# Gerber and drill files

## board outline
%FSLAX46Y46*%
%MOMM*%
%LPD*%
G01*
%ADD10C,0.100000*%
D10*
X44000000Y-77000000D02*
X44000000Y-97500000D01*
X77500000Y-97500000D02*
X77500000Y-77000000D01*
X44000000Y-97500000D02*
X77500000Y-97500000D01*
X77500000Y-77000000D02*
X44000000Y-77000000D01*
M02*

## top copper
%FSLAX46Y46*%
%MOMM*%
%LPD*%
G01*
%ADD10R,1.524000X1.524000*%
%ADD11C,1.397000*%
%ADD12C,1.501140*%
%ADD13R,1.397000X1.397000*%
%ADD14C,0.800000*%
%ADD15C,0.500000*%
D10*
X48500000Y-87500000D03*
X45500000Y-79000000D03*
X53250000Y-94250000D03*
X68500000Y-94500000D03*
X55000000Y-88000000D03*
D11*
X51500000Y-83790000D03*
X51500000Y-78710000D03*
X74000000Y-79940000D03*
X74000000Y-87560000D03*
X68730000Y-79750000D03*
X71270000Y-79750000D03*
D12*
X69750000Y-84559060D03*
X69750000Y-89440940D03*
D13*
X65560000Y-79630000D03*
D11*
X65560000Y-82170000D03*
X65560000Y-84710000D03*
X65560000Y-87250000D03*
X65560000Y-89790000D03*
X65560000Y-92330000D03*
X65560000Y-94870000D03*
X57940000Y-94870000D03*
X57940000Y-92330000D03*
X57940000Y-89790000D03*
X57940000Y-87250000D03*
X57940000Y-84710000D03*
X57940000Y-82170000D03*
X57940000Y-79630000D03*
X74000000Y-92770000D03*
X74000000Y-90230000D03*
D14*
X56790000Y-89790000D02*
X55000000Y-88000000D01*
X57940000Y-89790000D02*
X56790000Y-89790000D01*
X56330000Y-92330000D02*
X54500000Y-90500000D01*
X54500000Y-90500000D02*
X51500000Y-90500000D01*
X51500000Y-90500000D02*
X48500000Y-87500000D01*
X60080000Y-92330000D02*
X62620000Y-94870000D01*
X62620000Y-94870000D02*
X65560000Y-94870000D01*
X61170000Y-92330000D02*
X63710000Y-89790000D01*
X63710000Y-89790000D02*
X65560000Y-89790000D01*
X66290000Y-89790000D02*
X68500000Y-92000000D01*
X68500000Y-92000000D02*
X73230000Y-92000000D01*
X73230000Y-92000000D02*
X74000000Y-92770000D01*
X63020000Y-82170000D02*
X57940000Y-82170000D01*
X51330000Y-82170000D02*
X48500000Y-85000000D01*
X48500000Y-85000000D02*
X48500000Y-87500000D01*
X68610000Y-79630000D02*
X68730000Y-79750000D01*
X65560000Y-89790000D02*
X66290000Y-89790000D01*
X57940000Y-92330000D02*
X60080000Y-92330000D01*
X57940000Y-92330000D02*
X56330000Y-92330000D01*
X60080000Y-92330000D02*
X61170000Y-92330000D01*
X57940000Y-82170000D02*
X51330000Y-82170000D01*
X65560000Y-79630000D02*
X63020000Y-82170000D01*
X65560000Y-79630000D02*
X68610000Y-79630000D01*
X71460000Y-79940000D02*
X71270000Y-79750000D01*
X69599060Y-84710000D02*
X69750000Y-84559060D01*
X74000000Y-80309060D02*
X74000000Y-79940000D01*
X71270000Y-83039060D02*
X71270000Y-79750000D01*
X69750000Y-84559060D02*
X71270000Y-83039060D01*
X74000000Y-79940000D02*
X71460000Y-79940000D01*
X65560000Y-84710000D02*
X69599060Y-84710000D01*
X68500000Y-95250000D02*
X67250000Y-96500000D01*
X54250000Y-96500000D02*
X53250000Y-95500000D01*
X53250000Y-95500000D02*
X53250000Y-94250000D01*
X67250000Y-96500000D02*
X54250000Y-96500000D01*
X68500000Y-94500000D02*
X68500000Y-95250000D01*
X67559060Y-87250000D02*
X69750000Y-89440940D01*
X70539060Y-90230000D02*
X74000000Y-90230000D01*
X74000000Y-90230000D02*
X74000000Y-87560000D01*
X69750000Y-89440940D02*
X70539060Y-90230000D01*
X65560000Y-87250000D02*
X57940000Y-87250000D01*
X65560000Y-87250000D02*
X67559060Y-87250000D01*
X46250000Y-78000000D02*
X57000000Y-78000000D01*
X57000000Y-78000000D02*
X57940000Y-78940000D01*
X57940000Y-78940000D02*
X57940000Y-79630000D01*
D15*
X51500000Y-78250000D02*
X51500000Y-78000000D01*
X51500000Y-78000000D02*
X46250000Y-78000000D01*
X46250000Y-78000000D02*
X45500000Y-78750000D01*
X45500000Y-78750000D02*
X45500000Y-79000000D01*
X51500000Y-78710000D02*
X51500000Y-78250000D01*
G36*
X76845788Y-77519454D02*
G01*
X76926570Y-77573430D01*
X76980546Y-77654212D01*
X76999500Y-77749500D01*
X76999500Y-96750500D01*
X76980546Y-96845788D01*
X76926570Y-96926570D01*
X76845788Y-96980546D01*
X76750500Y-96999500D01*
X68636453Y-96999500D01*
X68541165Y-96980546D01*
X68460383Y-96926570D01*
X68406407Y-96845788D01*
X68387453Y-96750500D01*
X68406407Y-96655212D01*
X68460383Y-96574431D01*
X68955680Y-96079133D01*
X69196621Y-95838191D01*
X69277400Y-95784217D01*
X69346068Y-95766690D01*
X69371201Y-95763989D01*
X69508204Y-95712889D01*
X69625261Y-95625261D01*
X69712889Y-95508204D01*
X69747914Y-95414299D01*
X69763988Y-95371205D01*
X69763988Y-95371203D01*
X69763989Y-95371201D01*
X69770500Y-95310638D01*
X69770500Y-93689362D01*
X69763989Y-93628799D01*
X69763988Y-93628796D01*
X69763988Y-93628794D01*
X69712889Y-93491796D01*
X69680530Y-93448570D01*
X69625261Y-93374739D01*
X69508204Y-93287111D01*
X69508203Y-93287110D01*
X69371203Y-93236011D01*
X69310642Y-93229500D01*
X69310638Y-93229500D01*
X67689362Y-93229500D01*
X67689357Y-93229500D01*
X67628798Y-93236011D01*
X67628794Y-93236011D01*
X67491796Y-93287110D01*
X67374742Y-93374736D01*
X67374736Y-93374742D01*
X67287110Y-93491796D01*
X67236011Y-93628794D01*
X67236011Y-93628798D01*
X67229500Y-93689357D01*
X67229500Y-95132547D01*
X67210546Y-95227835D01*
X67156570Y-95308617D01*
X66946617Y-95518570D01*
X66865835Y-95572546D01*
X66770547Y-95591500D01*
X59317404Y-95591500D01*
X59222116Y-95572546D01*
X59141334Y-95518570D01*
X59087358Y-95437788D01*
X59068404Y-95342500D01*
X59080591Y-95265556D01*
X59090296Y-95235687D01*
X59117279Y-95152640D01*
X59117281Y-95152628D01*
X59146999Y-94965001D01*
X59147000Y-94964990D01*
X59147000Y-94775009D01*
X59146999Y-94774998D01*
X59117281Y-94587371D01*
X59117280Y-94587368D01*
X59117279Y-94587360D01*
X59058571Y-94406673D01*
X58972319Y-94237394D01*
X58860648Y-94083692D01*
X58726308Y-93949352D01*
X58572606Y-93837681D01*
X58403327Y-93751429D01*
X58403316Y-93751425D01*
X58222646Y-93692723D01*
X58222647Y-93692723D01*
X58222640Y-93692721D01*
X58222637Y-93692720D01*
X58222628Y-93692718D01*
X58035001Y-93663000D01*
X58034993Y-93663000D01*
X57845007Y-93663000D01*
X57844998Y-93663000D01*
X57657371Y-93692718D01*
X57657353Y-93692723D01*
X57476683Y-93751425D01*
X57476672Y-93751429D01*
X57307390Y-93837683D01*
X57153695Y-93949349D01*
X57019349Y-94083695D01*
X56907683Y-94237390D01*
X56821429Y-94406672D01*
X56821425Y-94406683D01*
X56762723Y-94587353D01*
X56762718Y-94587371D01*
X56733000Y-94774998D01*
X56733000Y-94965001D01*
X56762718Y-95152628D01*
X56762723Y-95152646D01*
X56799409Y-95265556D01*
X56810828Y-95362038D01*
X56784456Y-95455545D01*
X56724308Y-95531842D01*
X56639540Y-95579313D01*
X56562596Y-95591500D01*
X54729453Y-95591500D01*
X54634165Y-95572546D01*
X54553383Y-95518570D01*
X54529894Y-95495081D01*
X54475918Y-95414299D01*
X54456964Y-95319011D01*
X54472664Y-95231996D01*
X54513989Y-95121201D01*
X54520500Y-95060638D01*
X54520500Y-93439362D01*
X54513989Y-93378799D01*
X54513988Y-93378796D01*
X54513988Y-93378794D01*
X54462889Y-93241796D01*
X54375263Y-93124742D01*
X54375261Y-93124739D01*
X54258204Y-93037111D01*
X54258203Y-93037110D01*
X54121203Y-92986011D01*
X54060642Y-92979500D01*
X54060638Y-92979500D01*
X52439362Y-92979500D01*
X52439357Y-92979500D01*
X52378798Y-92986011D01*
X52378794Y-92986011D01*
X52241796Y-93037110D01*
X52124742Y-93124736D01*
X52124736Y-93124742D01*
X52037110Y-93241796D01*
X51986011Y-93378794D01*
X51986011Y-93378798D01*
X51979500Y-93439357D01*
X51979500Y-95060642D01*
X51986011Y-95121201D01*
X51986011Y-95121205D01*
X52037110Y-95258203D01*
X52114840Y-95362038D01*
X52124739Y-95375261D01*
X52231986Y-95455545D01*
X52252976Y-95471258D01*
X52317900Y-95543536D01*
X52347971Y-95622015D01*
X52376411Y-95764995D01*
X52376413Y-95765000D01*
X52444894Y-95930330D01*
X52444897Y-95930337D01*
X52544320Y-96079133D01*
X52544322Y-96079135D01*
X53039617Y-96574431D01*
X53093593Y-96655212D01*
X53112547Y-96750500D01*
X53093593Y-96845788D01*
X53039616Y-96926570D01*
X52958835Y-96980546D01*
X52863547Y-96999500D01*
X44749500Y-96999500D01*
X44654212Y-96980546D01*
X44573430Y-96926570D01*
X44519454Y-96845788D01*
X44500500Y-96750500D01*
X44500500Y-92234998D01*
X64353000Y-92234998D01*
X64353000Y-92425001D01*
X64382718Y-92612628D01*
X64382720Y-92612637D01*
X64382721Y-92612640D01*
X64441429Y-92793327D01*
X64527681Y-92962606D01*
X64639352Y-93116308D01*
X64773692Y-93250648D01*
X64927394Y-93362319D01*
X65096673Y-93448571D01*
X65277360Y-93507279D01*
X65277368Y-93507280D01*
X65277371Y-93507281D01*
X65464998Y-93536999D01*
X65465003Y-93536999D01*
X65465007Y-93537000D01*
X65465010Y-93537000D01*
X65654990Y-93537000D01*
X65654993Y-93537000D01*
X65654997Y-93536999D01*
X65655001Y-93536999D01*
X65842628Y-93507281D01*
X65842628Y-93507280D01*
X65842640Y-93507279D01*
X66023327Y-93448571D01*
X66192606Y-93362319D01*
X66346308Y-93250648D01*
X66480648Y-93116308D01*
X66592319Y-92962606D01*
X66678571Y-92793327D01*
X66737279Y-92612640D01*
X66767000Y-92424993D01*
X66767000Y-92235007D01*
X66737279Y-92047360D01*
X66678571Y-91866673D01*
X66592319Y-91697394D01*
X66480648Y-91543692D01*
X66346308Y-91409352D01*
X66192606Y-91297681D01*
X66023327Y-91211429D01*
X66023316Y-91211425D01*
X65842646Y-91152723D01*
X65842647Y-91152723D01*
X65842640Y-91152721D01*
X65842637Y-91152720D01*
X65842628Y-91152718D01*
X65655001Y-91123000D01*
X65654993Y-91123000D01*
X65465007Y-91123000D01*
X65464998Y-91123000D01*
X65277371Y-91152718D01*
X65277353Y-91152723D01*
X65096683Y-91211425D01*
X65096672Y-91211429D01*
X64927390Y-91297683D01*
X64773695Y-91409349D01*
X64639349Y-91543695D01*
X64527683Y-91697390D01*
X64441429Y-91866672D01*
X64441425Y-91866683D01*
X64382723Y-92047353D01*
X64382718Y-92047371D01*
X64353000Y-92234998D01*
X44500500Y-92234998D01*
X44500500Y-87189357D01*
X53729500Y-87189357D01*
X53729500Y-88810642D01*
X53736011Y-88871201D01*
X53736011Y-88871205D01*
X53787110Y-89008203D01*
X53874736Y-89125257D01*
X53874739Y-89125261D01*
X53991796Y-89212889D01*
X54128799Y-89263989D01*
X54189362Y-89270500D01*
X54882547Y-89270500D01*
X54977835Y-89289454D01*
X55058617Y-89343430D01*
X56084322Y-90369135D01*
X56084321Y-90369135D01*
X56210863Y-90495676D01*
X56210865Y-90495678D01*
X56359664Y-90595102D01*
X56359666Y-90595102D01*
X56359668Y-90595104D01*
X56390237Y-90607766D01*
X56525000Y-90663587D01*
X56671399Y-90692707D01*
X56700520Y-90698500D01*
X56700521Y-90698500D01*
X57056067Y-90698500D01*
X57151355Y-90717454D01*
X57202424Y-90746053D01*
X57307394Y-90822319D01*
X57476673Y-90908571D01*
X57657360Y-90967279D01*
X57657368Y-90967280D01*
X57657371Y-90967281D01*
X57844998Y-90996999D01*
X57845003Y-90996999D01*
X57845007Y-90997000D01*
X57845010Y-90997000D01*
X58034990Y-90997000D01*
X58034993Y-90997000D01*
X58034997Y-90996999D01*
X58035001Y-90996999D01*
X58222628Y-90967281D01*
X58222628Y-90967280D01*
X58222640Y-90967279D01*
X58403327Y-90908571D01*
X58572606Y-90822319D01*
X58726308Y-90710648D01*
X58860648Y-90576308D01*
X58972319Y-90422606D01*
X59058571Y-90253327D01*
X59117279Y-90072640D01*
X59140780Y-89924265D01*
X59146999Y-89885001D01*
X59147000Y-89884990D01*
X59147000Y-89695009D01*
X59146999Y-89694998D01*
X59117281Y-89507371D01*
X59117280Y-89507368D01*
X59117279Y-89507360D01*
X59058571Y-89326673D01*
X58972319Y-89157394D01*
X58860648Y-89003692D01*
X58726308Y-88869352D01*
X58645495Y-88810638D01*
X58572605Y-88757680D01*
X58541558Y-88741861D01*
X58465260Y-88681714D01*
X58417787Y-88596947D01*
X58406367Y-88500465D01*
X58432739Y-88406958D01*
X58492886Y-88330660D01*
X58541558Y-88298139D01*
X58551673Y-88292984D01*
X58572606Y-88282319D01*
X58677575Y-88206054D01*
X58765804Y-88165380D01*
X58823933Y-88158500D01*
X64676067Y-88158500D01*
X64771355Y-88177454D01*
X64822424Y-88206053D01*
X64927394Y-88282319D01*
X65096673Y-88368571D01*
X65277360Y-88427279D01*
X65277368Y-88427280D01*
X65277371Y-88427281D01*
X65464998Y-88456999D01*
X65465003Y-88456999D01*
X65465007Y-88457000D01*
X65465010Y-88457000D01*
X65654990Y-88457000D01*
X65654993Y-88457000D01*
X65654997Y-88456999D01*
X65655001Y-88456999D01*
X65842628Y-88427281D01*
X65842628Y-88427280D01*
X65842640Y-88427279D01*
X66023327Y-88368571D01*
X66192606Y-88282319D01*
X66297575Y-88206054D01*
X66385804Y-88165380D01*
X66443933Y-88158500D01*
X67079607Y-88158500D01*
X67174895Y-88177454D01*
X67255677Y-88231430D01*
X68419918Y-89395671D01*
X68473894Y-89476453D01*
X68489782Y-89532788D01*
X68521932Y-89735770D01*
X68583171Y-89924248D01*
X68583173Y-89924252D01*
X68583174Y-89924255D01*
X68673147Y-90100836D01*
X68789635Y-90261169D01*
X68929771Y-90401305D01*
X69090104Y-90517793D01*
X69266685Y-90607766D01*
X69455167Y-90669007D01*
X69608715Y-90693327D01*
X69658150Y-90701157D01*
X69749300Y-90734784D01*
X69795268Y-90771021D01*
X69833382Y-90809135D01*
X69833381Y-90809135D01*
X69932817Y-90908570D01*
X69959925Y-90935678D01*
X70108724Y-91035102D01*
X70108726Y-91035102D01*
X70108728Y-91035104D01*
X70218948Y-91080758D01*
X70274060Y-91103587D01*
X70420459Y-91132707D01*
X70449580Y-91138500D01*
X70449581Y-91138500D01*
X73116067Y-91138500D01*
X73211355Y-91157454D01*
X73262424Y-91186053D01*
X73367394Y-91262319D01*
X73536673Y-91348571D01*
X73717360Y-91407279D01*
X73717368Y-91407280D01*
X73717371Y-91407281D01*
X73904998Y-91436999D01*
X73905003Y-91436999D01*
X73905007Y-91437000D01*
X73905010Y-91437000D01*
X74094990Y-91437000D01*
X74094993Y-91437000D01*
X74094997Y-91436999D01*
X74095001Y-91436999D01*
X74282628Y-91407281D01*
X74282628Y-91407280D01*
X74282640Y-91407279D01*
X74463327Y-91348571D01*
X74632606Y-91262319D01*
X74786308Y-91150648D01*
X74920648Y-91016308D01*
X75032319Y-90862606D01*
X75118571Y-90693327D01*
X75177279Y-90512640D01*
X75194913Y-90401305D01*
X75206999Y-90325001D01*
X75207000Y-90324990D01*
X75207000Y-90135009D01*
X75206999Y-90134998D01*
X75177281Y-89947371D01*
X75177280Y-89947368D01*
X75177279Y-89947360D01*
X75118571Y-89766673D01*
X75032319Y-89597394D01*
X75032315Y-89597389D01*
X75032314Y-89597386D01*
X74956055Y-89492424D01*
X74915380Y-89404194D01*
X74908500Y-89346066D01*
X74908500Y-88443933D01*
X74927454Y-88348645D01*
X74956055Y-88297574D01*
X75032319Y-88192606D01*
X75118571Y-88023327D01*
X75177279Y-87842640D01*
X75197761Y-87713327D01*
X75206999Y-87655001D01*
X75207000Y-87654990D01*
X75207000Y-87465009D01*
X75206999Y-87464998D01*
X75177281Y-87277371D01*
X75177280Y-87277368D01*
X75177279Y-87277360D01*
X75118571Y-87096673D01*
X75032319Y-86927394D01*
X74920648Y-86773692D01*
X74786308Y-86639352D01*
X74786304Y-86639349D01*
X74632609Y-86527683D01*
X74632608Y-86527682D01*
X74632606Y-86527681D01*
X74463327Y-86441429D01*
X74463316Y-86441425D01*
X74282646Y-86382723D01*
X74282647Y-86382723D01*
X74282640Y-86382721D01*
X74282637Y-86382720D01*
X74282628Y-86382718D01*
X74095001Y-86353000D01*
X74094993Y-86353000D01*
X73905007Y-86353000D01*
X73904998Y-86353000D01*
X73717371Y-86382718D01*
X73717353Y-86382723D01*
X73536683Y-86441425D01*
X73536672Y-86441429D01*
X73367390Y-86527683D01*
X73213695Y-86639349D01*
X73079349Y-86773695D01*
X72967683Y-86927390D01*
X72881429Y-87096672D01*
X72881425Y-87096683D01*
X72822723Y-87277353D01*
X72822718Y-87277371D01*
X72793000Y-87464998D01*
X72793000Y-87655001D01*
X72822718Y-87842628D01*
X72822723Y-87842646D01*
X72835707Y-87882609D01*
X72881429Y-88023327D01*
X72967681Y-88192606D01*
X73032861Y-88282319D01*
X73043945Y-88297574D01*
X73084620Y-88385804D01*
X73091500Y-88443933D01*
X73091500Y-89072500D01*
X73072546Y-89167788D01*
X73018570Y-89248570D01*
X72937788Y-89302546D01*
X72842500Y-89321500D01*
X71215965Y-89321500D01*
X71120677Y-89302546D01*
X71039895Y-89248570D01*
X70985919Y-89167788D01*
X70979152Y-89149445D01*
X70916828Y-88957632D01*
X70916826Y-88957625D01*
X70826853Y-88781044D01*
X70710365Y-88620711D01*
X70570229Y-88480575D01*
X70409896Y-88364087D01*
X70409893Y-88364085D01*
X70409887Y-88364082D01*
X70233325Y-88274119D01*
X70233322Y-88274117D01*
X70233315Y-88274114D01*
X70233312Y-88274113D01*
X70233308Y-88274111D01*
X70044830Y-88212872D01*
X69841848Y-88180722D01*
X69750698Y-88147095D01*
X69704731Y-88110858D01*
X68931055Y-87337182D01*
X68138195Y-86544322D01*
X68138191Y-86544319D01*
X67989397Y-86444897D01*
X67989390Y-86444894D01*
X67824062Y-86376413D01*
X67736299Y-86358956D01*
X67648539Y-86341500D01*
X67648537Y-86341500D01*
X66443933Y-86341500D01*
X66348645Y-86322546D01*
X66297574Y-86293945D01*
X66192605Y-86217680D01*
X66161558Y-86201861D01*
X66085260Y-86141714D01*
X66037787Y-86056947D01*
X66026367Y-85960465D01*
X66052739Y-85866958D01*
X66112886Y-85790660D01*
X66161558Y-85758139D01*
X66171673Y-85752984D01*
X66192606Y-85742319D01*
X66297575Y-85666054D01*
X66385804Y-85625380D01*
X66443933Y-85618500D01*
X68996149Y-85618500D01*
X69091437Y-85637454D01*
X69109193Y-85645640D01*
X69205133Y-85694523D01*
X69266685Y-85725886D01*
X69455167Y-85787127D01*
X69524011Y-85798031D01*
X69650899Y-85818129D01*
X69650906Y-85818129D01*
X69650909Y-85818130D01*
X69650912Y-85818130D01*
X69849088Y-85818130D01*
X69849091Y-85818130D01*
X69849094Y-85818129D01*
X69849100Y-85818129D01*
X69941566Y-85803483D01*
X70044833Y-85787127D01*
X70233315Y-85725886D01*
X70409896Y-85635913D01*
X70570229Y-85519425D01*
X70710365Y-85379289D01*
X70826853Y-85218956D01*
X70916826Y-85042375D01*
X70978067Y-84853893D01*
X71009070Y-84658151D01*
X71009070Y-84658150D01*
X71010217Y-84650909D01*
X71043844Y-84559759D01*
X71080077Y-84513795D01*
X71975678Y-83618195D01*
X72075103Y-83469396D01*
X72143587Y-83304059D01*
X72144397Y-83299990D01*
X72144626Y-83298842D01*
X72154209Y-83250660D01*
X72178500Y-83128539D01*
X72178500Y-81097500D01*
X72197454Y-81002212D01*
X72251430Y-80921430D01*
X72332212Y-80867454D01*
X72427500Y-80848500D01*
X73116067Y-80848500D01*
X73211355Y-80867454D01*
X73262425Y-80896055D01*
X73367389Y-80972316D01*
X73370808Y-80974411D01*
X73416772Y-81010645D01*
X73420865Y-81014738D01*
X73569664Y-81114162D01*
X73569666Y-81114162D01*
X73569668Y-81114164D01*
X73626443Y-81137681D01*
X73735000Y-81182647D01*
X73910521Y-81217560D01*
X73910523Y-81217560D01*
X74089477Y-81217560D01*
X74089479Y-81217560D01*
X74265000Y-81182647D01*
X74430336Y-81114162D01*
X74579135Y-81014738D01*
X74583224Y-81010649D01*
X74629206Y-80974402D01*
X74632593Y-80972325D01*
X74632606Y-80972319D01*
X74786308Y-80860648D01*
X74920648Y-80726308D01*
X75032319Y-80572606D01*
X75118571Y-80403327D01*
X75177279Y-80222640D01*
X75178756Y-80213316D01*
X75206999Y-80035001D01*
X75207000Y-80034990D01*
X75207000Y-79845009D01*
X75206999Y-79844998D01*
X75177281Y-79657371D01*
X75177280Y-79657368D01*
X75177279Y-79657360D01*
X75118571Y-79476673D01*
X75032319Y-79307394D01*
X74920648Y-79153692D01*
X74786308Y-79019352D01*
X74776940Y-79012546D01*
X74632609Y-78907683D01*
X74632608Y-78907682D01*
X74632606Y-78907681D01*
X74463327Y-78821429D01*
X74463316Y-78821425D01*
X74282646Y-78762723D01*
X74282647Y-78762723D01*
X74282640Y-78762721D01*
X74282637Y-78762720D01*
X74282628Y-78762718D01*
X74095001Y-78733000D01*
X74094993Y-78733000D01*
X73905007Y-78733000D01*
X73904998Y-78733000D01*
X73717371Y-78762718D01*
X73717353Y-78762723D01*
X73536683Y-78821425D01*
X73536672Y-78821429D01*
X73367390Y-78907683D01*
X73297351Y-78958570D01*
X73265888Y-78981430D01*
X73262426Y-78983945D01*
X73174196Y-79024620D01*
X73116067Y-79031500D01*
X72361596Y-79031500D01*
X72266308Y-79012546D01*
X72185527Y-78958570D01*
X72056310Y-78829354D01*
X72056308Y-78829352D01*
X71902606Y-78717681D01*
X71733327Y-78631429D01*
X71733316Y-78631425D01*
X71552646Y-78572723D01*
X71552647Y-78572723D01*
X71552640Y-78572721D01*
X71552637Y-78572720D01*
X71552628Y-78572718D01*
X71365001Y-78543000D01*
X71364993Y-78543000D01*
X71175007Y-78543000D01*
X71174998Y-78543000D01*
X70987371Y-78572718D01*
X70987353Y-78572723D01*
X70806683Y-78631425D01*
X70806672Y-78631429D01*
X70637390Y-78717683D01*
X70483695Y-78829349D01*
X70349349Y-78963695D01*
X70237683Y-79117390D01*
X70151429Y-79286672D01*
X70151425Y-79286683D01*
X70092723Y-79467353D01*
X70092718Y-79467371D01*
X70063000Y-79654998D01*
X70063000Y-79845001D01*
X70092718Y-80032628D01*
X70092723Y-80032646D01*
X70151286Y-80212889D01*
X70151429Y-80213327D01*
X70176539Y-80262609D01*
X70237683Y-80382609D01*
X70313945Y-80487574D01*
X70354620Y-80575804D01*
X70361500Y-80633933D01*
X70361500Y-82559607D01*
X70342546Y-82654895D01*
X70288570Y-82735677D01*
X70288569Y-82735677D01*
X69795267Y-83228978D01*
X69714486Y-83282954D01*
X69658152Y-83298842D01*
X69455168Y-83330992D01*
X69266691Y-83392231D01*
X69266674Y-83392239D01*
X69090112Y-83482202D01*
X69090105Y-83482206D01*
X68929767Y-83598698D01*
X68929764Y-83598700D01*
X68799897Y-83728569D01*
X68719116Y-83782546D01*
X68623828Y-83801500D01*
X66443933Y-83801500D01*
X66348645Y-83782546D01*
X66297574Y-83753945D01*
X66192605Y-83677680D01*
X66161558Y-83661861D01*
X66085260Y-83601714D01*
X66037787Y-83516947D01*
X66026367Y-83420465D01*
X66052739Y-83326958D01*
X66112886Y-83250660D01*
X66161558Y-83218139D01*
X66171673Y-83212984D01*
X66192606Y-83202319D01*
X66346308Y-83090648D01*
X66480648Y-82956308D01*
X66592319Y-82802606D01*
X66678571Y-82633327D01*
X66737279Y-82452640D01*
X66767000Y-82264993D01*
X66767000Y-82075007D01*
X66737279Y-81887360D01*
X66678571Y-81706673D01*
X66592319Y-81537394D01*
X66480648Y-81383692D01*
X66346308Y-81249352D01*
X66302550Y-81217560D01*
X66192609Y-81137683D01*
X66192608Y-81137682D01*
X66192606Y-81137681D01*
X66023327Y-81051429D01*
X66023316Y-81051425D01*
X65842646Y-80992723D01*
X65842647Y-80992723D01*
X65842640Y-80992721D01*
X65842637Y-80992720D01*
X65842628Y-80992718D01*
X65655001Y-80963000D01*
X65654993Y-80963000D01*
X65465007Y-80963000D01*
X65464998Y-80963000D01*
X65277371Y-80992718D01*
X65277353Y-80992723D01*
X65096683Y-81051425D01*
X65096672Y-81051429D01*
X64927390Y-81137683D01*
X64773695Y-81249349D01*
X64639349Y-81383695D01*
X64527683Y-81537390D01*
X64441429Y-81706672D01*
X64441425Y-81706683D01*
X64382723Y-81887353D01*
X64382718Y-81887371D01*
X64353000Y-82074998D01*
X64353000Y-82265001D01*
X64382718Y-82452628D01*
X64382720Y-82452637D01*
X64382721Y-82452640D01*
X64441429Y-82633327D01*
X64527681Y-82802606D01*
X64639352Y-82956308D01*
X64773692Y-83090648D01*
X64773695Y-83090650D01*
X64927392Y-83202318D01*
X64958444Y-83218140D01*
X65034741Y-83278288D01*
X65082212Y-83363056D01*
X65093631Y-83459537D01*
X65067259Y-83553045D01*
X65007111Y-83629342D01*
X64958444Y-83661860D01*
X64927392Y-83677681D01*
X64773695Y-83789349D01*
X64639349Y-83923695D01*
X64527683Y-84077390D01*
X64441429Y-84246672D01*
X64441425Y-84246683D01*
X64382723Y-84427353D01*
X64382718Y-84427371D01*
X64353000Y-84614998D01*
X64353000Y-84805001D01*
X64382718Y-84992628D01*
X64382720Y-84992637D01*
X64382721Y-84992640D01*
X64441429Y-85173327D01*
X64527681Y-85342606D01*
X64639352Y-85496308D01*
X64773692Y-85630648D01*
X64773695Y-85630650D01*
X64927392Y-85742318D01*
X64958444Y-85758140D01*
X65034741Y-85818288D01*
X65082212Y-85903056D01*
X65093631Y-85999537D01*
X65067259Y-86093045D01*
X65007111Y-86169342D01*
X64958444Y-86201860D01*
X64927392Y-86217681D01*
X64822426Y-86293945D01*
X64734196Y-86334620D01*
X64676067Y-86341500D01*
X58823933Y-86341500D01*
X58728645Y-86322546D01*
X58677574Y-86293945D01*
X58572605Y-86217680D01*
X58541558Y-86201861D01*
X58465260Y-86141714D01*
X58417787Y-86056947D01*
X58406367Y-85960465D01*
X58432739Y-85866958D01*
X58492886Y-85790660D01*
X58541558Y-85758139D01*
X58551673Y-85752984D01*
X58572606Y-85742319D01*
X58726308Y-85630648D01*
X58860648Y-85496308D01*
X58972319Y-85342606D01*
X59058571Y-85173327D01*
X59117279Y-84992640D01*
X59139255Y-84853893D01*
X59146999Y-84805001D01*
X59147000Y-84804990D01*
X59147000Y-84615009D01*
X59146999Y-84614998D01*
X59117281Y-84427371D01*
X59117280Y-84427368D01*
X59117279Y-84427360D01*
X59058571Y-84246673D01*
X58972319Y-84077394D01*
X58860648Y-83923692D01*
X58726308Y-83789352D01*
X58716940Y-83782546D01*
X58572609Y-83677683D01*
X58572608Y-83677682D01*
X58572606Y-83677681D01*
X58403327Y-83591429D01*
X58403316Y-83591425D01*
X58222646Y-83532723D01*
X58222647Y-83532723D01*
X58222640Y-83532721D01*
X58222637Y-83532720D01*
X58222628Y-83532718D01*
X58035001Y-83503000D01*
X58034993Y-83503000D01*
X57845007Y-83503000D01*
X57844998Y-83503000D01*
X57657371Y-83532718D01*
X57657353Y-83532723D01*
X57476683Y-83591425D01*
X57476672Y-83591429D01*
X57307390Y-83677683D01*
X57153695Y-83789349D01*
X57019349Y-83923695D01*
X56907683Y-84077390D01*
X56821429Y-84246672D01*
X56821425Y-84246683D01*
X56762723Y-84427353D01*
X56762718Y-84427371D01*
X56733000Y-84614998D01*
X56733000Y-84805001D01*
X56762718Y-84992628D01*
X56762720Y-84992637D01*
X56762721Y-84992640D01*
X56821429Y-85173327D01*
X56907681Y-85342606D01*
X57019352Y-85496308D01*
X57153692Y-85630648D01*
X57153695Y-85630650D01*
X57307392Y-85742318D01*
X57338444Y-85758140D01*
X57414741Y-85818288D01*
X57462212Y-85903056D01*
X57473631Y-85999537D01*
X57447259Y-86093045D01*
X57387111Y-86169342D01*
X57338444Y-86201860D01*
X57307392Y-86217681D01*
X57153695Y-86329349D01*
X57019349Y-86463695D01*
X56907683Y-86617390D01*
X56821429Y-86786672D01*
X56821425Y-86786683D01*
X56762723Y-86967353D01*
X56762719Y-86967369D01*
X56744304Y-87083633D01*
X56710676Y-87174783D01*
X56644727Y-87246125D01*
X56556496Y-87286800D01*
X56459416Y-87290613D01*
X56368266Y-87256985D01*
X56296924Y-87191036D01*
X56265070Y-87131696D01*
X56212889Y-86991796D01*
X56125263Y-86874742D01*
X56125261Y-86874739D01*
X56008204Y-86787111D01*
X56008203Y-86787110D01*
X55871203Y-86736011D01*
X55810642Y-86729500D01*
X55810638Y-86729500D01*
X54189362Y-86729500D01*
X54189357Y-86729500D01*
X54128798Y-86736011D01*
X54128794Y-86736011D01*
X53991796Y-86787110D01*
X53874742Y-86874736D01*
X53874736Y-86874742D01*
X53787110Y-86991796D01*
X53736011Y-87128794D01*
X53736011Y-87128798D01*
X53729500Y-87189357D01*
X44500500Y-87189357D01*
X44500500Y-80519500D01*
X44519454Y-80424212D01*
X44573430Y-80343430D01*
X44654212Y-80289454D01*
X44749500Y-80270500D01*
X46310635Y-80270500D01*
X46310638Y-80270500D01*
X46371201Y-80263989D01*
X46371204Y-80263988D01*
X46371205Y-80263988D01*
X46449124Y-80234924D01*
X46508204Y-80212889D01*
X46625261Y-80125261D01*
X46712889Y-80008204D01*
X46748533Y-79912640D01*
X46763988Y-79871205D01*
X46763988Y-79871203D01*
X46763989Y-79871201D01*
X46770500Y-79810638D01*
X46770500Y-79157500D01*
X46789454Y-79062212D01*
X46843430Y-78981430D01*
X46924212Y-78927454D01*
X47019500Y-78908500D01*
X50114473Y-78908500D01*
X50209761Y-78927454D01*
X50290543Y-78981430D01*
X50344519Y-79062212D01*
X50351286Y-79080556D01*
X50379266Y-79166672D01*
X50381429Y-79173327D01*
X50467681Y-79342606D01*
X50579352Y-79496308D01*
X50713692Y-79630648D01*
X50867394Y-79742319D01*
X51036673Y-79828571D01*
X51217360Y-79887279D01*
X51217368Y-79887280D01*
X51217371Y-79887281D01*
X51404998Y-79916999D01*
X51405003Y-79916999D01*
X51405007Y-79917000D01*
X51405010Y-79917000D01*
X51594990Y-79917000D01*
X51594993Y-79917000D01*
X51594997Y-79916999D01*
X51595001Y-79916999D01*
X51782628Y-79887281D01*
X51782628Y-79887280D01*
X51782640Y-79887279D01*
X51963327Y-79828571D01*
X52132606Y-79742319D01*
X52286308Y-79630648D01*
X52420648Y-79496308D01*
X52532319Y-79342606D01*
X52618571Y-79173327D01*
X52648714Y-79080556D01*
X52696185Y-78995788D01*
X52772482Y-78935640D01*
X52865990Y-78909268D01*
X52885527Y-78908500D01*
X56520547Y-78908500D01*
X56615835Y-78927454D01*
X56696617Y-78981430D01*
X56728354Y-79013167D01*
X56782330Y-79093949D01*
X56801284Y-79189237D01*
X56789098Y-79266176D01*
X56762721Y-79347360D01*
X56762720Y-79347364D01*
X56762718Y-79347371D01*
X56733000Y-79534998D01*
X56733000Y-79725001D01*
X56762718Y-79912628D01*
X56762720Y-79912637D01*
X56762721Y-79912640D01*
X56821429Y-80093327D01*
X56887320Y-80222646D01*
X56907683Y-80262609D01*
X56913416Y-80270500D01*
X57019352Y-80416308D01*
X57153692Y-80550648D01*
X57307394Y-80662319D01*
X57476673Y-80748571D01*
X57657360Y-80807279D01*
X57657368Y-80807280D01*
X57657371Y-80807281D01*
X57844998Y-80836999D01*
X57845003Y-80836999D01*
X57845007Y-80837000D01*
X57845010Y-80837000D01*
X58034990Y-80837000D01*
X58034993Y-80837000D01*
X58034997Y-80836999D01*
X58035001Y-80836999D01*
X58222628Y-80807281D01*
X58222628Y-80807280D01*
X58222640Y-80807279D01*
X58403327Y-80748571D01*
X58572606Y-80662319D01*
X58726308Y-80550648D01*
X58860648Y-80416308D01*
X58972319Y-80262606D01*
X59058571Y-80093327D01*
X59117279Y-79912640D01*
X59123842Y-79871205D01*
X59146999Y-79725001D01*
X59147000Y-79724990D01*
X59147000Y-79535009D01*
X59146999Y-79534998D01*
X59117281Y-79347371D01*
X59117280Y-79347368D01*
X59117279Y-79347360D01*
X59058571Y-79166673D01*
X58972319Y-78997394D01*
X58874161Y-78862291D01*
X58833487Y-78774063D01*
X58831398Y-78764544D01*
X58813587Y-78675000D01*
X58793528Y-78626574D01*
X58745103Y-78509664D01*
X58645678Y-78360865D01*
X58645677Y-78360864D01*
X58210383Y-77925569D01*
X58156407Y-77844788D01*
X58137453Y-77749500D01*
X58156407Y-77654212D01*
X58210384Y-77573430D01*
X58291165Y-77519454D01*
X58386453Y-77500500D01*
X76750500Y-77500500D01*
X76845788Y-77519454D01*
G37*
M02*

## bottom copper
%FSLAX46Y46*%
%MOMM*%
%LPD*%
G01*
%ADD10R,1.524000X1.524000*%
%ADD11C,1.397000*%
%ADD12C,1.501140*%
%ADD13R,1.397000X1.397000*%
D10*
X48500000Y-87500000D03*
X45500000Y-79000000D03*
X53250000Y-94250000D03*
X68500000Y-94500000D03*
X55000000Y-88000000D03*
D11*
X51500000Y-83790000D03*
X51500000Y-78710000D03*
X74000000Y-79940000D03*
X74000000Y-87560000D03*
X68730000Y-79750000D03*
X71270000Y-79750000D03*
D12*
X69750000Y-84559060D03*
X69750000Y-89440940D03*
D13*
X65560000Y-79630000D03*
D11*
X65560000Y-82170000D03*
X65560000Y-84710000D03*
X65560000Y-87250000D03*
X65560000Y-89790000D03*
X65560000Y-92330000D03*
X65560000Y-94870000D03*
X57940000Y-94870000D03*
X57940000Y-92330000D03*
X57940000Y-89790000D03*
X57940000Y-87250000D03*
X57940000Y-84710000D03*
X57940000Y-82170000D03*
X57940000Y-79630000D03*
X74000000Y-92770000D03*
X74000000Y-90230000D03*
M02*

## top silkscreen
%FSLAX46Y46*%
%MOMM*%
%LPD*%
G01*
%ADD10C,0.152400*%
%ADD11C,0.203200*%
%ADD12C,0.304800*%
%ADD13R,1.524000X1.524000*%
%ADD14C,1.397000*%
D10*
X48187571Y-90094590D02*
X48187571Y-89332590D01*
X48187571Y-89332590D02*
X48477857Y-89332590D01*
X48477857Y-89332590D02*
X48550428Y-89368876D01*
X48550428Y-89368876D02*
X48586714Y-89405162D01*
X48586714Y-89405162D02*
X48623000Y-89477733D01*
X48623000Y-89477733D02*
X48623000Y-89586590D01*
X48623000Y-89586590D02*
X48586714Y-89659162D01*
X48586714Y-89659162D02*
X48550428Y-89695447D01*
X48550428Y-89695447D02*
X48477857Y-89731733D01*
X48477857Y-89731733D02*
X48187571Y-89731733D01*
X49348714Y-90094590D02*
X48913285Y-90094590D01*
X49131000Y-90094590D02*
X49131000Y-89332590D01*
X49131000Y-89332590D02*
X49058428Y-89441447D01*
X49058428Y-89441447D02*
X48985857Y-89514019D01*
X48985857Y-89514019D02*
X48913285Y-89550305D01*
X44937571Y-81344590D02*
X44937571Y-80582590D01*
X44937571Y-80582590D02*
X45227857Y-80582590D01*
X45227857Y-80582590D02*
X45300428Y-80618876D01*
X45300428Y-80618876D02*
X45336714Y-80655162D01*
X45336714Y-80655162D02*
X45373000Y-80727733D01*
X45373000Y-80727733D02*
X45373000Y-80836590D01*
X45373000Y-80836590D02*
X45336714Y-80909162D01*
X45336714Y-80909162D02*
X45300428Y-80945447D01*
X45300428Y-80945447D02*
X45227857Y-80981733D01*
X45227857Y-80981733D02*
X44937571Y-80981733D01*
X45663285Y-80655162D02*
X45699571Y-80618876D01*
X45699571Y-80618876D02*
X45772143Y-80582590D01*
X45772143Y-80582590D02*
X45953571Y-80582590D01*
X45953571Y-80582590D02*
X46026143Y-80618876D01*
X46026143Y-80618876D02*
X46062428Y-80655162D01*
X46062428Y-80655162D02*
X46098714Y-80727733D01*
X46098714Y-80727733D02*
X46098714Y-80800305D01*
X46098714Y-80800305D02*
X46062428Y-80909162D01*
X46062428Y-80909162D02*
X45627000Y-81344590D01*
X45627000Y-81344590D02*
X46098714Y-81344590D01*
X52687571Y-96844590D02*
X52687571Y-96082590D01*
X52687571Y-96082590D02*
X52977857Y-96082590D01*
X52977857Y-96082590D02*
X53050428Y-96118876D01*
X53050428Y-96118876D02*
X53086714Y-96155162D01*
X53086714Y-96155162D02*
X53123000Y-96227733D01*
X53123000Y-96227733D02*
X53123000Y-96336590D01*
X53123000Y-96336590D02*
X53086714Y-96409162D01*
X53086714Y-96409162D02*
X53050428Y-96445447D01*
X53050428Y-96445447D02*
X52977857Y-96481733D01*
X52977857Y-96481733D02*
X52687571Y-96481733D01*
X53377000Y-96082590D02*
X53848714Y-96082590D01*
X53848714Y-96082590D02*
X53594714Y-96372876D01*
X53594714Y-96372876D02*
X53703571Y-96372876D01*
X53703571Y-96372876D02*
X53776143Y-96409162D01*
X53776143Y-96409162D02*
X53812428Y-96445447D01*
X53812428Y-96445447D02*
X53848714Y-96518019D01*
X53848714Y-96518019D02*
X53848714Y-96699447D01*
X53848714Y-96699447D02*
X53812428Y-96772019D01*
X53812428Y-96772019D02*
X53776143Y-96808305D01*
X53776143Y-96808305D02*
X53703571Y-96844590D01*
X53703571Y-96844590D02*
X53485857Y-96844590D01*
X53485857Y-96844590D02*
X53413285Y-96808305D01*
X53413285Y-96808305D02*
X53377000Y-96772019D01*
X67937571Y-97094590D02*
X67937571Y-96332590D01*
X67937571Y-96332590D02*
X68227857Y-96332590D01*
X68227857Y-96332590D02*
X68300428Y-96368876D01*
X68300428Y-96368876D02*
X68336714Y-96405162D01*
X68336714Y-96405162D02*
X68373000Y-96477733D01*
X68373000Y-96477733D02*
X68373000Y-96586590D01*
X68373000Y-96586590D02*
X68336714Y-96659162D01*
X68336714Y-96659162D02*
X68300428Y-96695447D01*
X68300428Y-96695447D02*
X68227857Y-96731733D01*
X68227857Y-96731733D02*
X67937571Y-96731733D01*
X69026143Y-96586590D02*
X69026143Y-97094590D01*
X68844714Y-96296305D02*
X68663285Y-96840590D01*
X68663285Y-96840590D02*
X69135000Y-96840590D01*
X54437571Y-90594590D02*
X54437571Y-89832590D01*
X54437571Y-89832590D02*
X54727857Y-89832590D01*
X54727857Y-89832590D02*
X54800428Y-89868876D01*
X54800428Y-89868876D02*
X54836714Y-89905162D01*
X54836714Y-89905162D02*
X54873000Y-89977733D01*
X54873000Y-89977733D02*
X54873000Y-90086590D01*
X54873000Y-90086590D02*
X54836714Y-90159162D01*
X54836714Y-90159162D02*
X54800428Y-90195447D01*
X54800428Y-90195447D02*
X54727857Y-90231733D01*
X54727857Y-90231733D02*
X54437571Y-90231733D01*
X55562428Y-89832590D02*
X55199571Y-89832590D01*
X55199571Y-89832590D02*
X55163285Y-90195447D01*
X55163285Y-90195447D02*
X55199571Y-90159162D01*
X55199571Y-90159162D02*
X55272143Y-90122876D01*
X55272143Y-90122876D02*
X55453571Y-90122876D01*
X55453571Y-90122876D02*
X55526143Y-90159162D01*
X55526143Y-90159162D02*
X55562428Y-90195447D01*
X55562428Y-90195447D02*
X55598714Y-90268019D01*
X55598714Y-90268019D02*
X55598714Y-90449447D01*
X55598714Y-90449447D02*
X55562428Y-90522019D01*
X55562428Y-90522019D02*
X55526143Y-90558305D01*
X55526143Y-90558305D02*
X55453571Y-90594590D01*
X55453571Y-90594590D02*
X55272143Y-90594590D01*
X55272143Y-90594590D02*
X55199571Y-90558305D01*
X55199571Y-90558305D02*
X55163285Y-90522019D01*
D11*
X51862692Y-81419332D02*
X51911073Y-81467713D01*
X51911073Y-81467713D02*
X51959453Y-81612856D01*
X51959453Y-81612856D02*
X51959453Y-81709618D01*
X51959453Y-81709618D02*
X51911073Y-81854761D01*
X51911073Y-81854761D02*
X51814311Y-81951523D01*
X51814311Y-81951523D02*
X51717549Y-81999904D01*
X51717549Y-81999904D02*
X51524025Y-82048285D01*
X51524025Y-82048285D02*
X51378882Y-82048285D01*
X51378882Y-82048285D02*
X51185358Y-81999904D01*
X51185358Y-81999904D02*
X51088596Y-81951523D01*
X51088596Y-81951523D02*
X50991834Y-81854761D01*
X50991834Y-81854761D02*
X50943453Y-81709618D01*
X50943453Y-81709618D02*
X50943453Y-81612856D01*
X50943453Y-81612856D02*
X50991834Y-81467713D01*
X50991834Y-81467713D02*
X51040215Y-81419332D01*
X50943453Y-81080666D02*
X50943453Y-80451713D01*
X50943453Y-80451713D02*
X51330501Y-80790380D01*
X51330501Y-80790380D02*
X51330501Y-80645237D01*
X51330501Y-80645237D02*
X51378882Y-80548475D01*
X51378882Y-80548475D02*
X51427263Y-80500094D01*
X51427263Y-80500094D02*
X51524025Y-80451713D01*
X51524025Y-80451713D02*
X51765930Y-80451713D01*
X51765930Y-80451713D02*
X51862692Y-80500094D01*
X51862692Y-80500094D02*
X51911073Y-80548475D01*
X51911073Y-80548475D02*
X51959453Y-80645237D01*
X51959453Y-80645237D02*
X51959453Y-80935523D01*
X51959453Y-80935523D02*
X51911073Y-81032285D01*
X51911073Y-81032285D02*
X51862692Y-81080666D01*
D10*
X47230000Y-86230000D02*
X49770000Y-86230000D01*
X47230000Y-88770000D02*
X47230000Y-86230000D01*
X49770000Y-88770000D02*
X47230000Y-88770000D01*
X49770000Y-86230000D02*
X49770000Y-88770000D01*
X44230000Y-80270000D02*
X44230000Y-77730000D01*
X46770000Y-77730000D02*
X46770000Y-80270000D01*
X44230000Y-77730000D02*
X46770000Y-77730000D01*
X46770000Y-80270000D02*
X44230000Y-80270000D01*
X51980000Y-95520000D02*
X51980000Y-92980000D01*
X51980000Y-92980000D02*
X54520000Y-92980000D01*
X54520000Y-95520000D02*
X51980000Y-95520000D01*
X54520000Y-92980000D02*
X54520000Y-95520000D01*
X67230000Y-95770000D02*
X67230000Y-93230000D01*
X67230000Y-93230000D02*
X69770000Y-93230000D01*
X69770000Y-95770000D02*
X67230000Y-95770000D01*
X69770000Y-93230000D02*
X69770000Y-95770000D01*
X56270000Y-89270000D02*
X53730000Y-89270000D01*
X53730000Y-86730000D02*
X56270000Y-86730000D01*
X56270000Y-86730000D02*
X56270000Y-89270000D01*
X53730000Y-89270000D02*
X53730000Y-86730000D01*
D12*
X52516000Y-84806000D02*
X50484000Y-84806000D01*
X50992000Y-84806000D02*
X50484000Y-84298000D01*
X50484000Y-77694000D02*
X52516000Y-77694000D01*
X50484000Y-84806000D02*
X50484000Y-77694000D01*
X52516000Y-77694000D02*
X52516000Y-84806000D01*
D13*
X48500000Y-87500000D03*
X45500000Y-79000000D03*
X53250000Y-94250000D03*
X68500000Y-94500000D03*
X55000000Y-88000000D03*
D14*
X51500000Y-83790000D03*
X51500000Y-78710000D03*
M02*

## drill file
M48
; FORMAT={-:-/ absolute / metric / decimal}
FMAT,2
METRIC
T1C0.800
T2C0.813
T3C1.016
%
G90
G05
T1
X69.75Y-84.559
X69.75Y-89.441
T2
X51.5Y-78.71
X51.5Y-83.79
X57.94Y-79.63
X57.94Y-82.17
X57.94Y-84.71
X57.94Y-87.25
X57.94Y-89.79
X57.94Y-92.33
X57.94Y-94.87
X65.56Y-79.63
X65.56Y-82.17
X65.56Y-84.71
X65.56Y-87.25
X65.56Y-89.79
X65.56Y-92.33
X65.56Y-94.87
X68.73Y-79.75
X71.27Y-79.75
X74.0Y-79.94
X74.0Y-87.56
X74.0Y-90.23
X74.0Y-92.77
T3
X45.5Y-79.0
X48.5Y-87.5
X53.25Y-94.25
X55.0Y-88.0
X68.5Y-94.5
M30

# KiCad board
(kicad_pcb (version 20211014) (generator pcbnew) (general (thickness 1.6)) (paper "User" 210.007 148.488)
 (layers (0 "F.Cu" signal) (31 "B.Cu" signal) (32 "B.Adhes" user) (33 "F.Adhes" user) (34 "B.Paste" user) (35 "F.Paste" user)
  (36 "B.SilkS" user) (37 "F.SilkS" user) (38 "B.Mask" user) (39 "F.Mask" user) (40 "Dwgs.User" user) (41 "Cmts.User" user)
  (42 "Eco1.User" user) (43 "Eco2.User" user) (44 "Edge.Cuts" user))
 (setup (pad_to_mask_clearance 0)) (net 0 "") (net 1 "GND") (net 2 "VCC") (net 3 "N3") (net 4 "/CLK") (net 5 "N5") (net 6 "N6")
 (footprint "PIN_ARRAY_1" (layer "F.Cu") (at 48.5 87.5)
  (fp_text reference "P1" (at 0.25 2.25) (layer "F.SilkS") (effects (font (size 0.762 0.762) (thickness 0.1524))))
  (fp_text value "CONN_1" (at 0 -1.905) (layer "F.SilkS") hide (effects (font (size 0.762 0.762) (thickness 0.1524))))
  (fp_line (start -1.27 -1.27) (end 1.27 -1.27) (layer "F.SilkS") (width 0.1524))
  (fp_line (start -1.27 1.27) (end -1.27 -1.27) (layer "F.SilkS") (width 0.1524))
  (fp_line (start 1.27 1.27) (end -1.27 1.27) (layer "F.SilkS") (width 0.1524))
  (fp_line (start 1.27 -1.27) (end 1.27 1.27) (layer "F.SilkS") (width 0.1524))
  (pad "1" thru_hole rect locked (at 0 0) (size 1.524 1.524) (drill 1.016) (layers *.Cu *.Mask "F.SilkS") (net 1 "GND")))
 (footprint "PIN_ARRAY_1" (layer "F.Cu") (at 45.5 79)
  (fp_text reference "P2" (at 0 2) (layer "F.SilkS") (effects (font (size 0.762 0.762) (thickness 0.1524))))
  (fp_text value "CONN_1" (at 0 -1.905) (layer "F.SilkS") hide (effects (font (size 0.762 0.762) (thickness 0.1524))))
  (fp_line (start -1.27 1.27) (end -1.27 -1.27) (layer "F.SilkS") (width 0.1524))
  (fp_line (start 1.27 -1.27) (end 1.27 1.27) (layer "F.SilkS") (width 0.1524))
  (fp_line (start -1.27 -1.27) (end 1.27 -1.27) (layer "F.SilkS") (width 0.1524))
  (fp_line (start 1.27 1.27) (end -1.27 1.27) (layer "F.SilkS") (width 0.1524))
  (pad "1" thru_hole rect locked (at 0 0) (size 1.524 1.524) (drill 1.016) (layers *.Cu *.Mask "F.SilkS") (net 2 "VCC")))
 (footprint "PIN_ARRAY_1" (layer "F.Cu") (at 53.25 94.25)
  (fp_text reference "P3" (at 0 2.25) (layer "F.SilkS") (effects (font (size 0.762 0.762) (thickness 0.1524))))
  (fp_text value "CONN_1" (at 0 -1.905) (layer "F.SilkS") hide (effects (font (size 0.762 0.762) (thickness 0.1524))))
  (fp_line (start -1.27 1.27) (end -1.27 -1.27) (layer "F.SilkS") (width 0.1524))
  (fp_line (start -1.27 -1.27) (end 1.27 -1.27) (layer "F.SilkS") (width 0.1524))
  (fp_line (start 1.27 1.27) (end -1.27 1.27) (layer "F.SilkS") (width 0.1524))
  (fp_line (start 1.27 -1.27) (end 1.27 1.27) (layer "F.SilkS") (width 0.1524))
  (pad "1" thru_hole rect locked (at 0 0) (size 1.524 1.524) (drill 1.016) (layers *.Cu *.Mask "F.SilkS") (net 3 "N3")))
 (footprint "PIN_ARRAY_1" (layer "F.Cu") (at 68.5 94.5)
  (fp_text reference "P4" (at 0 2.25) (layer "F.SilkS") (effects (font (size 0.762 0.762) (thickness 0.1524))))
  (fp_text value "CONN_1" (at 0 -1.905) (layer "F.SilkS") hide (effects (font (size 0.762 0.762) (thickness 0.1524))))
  (fp_line (start -1.27 1.27) (end -1.27 -1.27) (layer "F.SilkS") (width 0.1524))
  (fp_line (start -1.27 -1.27) (end 1.27 -1.27) (layer "F.SilkS") (width 0.1524))
  (fp_line (start 1.27 1.27) (end -1.27 1.27) (layer "F.SilkS") (width 0.1524))
  (fp_line (start 1.27 -1.27) (end 1.27 1.27) (layer "F.SilkS") (width 0.1524))
  (pad "1" thru_hole rect locked (at 0 0) (size 1.524 1.524) (drill 1.016) (layers *.Cu *.Mask "F.SilkS") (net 3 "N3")))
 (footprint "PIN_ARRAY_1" (layer "F.Cu") (at 55 88)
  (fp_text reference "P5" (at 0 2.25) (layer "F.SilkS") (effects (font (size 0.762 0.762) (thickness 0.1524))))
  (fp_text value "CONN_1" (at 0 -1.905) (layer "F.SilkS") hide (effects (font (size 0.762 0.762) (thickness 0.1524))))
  (fp_line (start 1.27 1.27) (end -1.27 1.27) (layer "F.SilkS") (width 0.1524))
  (fp_line (start -1.27 -1.27) (end 1.27 -1.27) (layer "F.SilkS") (width 0.1524))
  (fp_line (start 1.27 -1.27) (end 1.27 1.27) (layer "F.SilkS") (width 0.1524))
  (fp_line (start -1.27 1.27) (end -1.27 -1.27) (layer "F.SilkS") (width 0.1524))
  (pad "1" thru_hole rect locked (at 0 0) (size 1.524 1.524) (drill 1.016) (layers *.Cu *.Mask "F.SilkS") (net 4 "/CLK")))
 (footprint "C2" (layer "F.Cu") (at 51.5 81.25 90)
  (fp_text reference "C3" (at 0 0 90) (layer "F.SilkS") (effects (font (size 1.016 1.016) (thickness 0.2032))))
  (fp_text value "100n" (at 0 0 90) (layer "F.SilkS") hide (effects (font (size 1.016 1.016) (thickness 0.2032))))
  (fp_line (start -3.556 1.016) (end -3.556 -1.016) (layer "F.SilkS") (width 0.3048))
  (fp_line (start -3.556 -0.508) (end -3.048 -1.016) (layer "F.SilkS") (width 0.3048))
  (fp_line (start 3.556 -1.016) (end 3.556 1.016) (layer "F.SilkS") (width 0.3048))
  (fp_line (start -3.556 -1.016) (end 3.556 -1.016) (layer "F.SilkS") (width 0.3048))
  (fp_line (start 3.556 1.016) (end -3.556 1.016) (layer "F.SilkS") (width 0.3048))
  (pad "1" thru_hole circle locked (at -2.54 0 90) (size 1.397 1.397) (drill 0.8128) (layers *.Cu *.Mask "F.SilkS") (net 1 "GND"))
  (pad "2" thru_hole circle locked (at 2.54 0 90) (size 1.397 1.397) (drill 0.8128) (layers *.Cu *.Mask "F.SilkS") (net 2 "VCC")))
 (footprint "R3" (layer "B.Cu") (at 74 83.75 -90) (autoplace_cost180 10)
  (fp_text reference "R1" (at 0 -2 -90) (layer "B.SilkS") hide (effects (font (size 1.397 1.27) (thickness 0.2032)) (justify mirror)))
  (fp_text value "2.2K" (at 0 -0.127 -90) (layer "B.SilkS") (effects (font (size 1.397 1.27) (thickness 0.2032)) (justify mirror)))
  (pad "1" thru_hole circle locked (at -3.81 0 270) (size 1.397 1.397) (drill 0.8128) (layers *.Cu *.Mask "B.SilkS") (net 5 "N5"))
  (pad "2" thru_hole circle locked (at 3.81 0 270) (size 1.397 1.397) (drill 0.8128) (layers *.Cu *.Mask "B.SilkS") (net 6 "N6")))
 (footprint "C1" (layer "B.Cu") (at 70 79.75)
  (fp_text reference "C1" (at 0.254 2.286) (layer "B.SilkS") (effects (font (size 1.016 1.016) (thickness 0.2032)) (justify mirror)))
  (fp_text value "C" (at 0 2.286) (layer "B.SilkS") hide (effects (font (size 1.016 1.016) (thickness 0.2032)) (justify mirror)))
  (pad "1" thru_hole circle locked (at -1.27 0) (size 1.397 1.397) (drill 0.8128) (layers *.Cu *.Mask "B.SilkS") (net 1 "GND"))
  (pad "2" thru_hole circle locked (at 1.27 0) (size 1.397 1.397) (drill 0.8128) (layers *.Cu *.Mask "B.SilkS") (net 5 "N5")))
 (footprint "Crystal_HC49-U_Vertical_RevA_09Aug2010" (layer "B.Cu") (at 69.75 87 -90)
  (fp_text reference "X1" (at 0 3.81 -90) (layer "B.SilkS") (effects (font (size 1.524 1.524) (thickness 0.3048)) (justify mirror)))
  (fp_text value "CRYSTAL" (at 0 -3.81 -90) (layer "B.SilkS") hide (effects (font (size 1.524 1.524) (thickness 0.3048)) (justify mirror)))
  (pad "1" thru_hole circle locked (at -2.44094 0 270) (size 1.50114 1.50114) (drill 0.8001) (layers *.Cu *.Mask "B.SilkS") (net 5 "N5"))
  (pad "2" thru_hole circle locked (at 2.44094 0 270) (size 1.50114 1.50114) (drill 0.8001) (layers *.Cu *.Mask "B.SilkS") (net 6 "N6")))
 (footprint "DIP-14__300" (layer "B.Cu") (at 61.75 87.25 -90)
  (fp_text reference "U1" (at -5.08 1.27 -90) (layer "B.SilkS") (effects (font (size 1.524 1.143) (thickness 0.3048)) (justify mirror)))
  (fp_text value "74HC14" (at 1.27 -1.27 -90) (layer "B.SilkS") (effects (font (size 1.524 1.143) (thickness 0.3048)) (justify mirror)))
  (pad "1" thru_hole rect locked (at -7.62 -3.81 270) (size 1.397 1.397) (drill 0.8128) (layers *.Cu *.Mask "B.SilkS") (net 1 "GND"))
  (pad "2" thru_hole circle locked (at -5.08 -3.81 270) (size 1.397 1.397) (drill 0.8128) (layers *.Cu *.Mask "B.SilkS"))
  (pad "3" thru_hole circle locked (at -2.54 -3.81 270) (size 1.397 1.397) (drill 0.8128) (layers *.Cu *.Mask "B.SilkS") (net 5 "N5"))
  (pad "4" thru_hole circle locked (at 0 -3.81 270) (size 1.397 1.397) (drill 0.8128) (layers *.Cu *.Mask "B.SilkS") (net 6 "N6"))
  (pad "5" thru_hole circle locked (at 2.54 -3.81 270) (size 1.397 1.397) (drill 0.8128) (layers *.Cu *.Mask "B.SilkS") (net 1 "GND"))
  (pad "6" thru_hole circle locked (at 5.08 -3.81 270) (size 1.397 1.397) (drill 0.8128) (layers *.Cu *.Mask "B.SilkS"))
  (pad "7" thru_hole circle locked (at 7.62 -3.81 270) (size 1.397 1.397) (drill 0.8128) (layers *.Cu *.Mask "B.SilkS") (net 1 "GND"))
  (pad "8" thru_hole circle locked (at 7.62 3.81 270) (size 1.397 1.397) (drill 0.8128) (layers *.Cu *.Mask "B.SilkS"))
  (pad "9" thru_hole circle locked (at 5.08 3.81 270) (size 1.397 1.397) (drill 0.8128) (layers *.Cu *.Mask "B.SilkS") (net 1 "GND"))
  (pad "10" thru_hole circle locked (at 2.54 3.81 270) (size 1.397 1.397) (drill 0.8128) (layers *.Cu *.Mask "B.SilkS") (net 4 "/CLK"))
  (pad "11" thru_hole circle locked (at 0 3.81 270) (size 1.397 1.397) (drill 0.8128) (layers *.Cu *.Mask "B.SilkS") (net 6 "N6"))
  (pad "12" thru_hole circle locked (at -2.54 3.81 270) (size 1.397 1.397) (drill 0.8128) (layers *.Cu *.Mask "B.SilkS"))
  (pad "13" thru_hole circle locked (at -5.08 3.81 270) (size 1.397 1.397) (drill 0.8128) (layers *.Cu *.Mask "B.SilkS") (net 1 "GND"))
  (pad "14" thru_hole circle locked (at -7.62 3.81 270) (size 1.397 1.397) (drill 0.8128) (layers *.Cu *.Mask "B.SilkS") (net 2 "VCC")))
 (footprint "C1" (layer "B.Cu") (at 74 91.5 90)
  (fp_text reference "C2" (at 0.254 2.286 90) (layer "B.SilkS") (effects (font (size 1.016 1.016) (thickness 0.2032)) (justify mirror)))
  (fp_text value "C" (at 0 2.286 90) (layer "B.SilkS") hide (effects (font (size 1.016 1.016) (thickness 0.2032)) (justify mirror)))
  (pad "1" thru_hole circle locked (at -1.27 0 90) (size 1.397 1.397) (drill 0.8128) (layers *.Cu *.Mask "B.SilkS") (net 1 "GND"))
  (pad "2" thru_hole circle locked (at 1.27 0 90) (size 1.397 1.397) (drill 0.8128) (layers *.Cu *.Mask "B.SilkS") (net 6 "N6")))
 (gr_line (start 44 77) (end 44 97.5) (layer "Edge.Cuts") (width 0.1))
 (gr_line (start 77.5 97.5) (end 77.5 77) (layer "Edge.Cuts") (width 0.1))
 (gr_line (start 44 97.5) (end 77.5 97.5) (layer "Edge.Cuts") (width 0.1))
 (gr_line (start 77.5 77) (end 44 77) (layer "Edge.Cuts") (width 0.1))
 (segment (start 56.79 89.79) (end 55 88) (width 0.8) (layer "F.Cu") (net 4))
 (segment (start 57.94 89.79) (end 56.79 89.79) (width 0.8) (layer "F.Cu") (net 4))
 (segment (start 56.33 92.33) (end 54.5 90.5) (width 0.8) (layer "F.Cu") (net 1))
 (segment (start 54.5 90.5) (end 51.5 90.5) (width 0.8) (layer "F.Cu") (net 1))
 (segment (start 51.5 90.5) (end 48.5 87.5) (width 0.8) (layer "F.Cu") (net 1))
 (segment (start 60.08 92.33) (end 62.62 94.87) (width 0.8) (layer "F.Cu") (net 1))
 (segment (start 62.62 94.87) (end 65.56 94.87) (width 0.8) (layer "F.Cu") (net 1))
 (segment (start 61.17 92.33) (end 63.71 89.79) (width 0.8) (layer "F.Cu") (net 1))
 (segment (start 63.71 89.79) (end 65.56 89.79) (width 0.8) (layer "F.Cu") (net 1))
 (segment (start 66.29 89.79) (end 68.5 92) (width 0.8) (layer "F.Cu") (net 1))
 (segment (start 68.5 92) (end 73.23 92) (width 0.8) (layer "F.Cu") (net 1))
 (segment (start 73.23 92) (end 74 92.77) (width 0.8) (layer "F.Cu") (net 1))
 (segment (start 63.02 82.17) (end 57.94 82.17) (width 0.8) (layer "F.Cu") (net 1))
 (segment (start 51.33 82.17) (end 48.5 85) (width 0.8) (layer "F.Cu") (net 1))
 (segment (start 48.5 85) (end 48.5 87.5) (width 0.8) (layer "F.Cu") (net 1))
 (segment (start 68.61 79.63) (end 68.73 79.75) (width 0.8) (layer "F.Cu") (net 1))
 (segment (start 65.56 89.79) (end 66.29 89.79) (width 0.8) (layer "F.Cu") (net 1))
 (segment (start 57.94 92.33) (end 60.08 92.33) (width 0.8) (layer "F.Cu") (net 1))
 (segment (start 57.94 92.33) (end 56.33 92.33) (width 0.8) (layer "F.Cu") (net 1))
 (segment (start 60.08 92.33) (end 61.17 92.33) (width 0.8) (layer "F.Cu") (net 1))
 (segment (start 57.94 82.17) (end 51.33 82.17) (width 0.8) (layer "F.Cu") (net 1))
 (segment (start 65.56 79.63) (end 63.02 82.17) (width 0.8) (layer "F.Cu") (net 1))
 (segment (start 65.56 79.63) (end 68.61 79.63) (width 0.8) (layer "F.Cu") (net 1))
 (segment (start 71.46 79.94) (end 71.27 79.75) (width 0.8) (layer "F.Cu") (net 5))
 (segment (start 69.59906 84.71) (end 69.75 84.55906) (width 0.8) (layer "F.Cu") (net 5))
 (segment (start 74 80.30906) (end 74 79.94) (width 0.8) (layer "F.Cu") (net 5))
 (segment (start 71.27 83.03906) (end 71.27 79.75) (width 0.8) (layer "F.Cu") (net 5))
 (segment (start 69.75 84.55906) (end 71.27 83.03906) (width 0.8) (layer "F.Cu") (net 5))
 (segment (start 74 79.94) (end 71.46 79.94) (width 0.8) (layer "F.Cu") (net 5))
 (segment (start 65.56 84.71) (end 69.59906 84.71) (width 0.8) (layer "F.Cu") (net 5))
 (segment (start 68.5 95.25) (end 67.25 96.5) (width 0.8) (layer "F.Cu") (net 3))
 (segment (start 54.25 96.5) (end 53.25 95.5) (width 0.8) (layer "F.Cu") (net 3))
 (segment (start 53.25 95.5) (end 53.25 94.25) (width 0.8) (layer "F.Cu") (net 3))
 (segment (start 67.25 96.5) (end 54.25 96.5) (width 0.8) (layer "F.Cu") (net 3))
 (segment (start 68.5 94.5) (end 68.5 95.25) (width 0.8) (layer "F.Cu") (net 3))
 (segment (start 67.55906 87.25) (end 69.75 89.44094) (width 0.8) (layer "F.Cu") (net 6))
 (segment (start 70.53906 90.23) (end 74 90.23) (width 0.8) (layer "F.Cu") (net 6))
 (segment (start 74 90.23) (end 74 87.56) (width 0.8) (layer "F.Cu") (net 6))
 (segment (start 69.75 89.44094) (end 70.53906 90.23) (width 0.8) (layer "F.Cu") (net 6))
 (segment (start 65.56 87.25) (end 57.94 87.25) (width 0.8) (layer "F.Cu") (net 6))
 (segment (start 65.56 87.25) (end 67.55906 87.25) (width 0.8) (layer "F.Cu") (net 6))
 (segment (start 46.25 78) (end 57 78) (width 0.8) (layer "F.Cu") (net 2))
 (segment (start 57 78) (end 57.94 78.94) (width 0.8) (layer "F.Cu") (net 2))
 (segment (start 57.94 78.94) (end 57.94 79.63) (width 0.8) (layer "F.Cu") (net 2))
 (segment (start 51.5 78.25) (end 51.5 78) (width 0.5) (layer "F.Cu") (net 2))
 (segment (start 51.5 78) (end 46.25 78) (width 0.5) (layer "F.Cu") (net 2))
 (segment (start 46.25 78) (end 45.5 78.75) (width 0.5) (layer "F.Cu") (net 2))
 (segment (start 45.5 78.75) (end 45.5 79) (width 0.5) (layer "F.Cu") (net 2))
 (segment (start 51.5 78.71) (end 51.5 78.25) (width 0.5) (layer "F.Cu") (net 2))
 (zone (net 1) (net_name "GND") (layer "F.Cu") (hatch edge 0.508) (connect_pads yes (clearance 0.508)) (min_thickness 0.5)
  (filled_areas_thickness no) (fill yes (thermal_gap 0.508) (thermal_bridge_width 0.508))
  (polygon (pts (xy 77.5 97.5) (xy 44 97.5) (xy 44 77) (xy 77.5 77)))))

